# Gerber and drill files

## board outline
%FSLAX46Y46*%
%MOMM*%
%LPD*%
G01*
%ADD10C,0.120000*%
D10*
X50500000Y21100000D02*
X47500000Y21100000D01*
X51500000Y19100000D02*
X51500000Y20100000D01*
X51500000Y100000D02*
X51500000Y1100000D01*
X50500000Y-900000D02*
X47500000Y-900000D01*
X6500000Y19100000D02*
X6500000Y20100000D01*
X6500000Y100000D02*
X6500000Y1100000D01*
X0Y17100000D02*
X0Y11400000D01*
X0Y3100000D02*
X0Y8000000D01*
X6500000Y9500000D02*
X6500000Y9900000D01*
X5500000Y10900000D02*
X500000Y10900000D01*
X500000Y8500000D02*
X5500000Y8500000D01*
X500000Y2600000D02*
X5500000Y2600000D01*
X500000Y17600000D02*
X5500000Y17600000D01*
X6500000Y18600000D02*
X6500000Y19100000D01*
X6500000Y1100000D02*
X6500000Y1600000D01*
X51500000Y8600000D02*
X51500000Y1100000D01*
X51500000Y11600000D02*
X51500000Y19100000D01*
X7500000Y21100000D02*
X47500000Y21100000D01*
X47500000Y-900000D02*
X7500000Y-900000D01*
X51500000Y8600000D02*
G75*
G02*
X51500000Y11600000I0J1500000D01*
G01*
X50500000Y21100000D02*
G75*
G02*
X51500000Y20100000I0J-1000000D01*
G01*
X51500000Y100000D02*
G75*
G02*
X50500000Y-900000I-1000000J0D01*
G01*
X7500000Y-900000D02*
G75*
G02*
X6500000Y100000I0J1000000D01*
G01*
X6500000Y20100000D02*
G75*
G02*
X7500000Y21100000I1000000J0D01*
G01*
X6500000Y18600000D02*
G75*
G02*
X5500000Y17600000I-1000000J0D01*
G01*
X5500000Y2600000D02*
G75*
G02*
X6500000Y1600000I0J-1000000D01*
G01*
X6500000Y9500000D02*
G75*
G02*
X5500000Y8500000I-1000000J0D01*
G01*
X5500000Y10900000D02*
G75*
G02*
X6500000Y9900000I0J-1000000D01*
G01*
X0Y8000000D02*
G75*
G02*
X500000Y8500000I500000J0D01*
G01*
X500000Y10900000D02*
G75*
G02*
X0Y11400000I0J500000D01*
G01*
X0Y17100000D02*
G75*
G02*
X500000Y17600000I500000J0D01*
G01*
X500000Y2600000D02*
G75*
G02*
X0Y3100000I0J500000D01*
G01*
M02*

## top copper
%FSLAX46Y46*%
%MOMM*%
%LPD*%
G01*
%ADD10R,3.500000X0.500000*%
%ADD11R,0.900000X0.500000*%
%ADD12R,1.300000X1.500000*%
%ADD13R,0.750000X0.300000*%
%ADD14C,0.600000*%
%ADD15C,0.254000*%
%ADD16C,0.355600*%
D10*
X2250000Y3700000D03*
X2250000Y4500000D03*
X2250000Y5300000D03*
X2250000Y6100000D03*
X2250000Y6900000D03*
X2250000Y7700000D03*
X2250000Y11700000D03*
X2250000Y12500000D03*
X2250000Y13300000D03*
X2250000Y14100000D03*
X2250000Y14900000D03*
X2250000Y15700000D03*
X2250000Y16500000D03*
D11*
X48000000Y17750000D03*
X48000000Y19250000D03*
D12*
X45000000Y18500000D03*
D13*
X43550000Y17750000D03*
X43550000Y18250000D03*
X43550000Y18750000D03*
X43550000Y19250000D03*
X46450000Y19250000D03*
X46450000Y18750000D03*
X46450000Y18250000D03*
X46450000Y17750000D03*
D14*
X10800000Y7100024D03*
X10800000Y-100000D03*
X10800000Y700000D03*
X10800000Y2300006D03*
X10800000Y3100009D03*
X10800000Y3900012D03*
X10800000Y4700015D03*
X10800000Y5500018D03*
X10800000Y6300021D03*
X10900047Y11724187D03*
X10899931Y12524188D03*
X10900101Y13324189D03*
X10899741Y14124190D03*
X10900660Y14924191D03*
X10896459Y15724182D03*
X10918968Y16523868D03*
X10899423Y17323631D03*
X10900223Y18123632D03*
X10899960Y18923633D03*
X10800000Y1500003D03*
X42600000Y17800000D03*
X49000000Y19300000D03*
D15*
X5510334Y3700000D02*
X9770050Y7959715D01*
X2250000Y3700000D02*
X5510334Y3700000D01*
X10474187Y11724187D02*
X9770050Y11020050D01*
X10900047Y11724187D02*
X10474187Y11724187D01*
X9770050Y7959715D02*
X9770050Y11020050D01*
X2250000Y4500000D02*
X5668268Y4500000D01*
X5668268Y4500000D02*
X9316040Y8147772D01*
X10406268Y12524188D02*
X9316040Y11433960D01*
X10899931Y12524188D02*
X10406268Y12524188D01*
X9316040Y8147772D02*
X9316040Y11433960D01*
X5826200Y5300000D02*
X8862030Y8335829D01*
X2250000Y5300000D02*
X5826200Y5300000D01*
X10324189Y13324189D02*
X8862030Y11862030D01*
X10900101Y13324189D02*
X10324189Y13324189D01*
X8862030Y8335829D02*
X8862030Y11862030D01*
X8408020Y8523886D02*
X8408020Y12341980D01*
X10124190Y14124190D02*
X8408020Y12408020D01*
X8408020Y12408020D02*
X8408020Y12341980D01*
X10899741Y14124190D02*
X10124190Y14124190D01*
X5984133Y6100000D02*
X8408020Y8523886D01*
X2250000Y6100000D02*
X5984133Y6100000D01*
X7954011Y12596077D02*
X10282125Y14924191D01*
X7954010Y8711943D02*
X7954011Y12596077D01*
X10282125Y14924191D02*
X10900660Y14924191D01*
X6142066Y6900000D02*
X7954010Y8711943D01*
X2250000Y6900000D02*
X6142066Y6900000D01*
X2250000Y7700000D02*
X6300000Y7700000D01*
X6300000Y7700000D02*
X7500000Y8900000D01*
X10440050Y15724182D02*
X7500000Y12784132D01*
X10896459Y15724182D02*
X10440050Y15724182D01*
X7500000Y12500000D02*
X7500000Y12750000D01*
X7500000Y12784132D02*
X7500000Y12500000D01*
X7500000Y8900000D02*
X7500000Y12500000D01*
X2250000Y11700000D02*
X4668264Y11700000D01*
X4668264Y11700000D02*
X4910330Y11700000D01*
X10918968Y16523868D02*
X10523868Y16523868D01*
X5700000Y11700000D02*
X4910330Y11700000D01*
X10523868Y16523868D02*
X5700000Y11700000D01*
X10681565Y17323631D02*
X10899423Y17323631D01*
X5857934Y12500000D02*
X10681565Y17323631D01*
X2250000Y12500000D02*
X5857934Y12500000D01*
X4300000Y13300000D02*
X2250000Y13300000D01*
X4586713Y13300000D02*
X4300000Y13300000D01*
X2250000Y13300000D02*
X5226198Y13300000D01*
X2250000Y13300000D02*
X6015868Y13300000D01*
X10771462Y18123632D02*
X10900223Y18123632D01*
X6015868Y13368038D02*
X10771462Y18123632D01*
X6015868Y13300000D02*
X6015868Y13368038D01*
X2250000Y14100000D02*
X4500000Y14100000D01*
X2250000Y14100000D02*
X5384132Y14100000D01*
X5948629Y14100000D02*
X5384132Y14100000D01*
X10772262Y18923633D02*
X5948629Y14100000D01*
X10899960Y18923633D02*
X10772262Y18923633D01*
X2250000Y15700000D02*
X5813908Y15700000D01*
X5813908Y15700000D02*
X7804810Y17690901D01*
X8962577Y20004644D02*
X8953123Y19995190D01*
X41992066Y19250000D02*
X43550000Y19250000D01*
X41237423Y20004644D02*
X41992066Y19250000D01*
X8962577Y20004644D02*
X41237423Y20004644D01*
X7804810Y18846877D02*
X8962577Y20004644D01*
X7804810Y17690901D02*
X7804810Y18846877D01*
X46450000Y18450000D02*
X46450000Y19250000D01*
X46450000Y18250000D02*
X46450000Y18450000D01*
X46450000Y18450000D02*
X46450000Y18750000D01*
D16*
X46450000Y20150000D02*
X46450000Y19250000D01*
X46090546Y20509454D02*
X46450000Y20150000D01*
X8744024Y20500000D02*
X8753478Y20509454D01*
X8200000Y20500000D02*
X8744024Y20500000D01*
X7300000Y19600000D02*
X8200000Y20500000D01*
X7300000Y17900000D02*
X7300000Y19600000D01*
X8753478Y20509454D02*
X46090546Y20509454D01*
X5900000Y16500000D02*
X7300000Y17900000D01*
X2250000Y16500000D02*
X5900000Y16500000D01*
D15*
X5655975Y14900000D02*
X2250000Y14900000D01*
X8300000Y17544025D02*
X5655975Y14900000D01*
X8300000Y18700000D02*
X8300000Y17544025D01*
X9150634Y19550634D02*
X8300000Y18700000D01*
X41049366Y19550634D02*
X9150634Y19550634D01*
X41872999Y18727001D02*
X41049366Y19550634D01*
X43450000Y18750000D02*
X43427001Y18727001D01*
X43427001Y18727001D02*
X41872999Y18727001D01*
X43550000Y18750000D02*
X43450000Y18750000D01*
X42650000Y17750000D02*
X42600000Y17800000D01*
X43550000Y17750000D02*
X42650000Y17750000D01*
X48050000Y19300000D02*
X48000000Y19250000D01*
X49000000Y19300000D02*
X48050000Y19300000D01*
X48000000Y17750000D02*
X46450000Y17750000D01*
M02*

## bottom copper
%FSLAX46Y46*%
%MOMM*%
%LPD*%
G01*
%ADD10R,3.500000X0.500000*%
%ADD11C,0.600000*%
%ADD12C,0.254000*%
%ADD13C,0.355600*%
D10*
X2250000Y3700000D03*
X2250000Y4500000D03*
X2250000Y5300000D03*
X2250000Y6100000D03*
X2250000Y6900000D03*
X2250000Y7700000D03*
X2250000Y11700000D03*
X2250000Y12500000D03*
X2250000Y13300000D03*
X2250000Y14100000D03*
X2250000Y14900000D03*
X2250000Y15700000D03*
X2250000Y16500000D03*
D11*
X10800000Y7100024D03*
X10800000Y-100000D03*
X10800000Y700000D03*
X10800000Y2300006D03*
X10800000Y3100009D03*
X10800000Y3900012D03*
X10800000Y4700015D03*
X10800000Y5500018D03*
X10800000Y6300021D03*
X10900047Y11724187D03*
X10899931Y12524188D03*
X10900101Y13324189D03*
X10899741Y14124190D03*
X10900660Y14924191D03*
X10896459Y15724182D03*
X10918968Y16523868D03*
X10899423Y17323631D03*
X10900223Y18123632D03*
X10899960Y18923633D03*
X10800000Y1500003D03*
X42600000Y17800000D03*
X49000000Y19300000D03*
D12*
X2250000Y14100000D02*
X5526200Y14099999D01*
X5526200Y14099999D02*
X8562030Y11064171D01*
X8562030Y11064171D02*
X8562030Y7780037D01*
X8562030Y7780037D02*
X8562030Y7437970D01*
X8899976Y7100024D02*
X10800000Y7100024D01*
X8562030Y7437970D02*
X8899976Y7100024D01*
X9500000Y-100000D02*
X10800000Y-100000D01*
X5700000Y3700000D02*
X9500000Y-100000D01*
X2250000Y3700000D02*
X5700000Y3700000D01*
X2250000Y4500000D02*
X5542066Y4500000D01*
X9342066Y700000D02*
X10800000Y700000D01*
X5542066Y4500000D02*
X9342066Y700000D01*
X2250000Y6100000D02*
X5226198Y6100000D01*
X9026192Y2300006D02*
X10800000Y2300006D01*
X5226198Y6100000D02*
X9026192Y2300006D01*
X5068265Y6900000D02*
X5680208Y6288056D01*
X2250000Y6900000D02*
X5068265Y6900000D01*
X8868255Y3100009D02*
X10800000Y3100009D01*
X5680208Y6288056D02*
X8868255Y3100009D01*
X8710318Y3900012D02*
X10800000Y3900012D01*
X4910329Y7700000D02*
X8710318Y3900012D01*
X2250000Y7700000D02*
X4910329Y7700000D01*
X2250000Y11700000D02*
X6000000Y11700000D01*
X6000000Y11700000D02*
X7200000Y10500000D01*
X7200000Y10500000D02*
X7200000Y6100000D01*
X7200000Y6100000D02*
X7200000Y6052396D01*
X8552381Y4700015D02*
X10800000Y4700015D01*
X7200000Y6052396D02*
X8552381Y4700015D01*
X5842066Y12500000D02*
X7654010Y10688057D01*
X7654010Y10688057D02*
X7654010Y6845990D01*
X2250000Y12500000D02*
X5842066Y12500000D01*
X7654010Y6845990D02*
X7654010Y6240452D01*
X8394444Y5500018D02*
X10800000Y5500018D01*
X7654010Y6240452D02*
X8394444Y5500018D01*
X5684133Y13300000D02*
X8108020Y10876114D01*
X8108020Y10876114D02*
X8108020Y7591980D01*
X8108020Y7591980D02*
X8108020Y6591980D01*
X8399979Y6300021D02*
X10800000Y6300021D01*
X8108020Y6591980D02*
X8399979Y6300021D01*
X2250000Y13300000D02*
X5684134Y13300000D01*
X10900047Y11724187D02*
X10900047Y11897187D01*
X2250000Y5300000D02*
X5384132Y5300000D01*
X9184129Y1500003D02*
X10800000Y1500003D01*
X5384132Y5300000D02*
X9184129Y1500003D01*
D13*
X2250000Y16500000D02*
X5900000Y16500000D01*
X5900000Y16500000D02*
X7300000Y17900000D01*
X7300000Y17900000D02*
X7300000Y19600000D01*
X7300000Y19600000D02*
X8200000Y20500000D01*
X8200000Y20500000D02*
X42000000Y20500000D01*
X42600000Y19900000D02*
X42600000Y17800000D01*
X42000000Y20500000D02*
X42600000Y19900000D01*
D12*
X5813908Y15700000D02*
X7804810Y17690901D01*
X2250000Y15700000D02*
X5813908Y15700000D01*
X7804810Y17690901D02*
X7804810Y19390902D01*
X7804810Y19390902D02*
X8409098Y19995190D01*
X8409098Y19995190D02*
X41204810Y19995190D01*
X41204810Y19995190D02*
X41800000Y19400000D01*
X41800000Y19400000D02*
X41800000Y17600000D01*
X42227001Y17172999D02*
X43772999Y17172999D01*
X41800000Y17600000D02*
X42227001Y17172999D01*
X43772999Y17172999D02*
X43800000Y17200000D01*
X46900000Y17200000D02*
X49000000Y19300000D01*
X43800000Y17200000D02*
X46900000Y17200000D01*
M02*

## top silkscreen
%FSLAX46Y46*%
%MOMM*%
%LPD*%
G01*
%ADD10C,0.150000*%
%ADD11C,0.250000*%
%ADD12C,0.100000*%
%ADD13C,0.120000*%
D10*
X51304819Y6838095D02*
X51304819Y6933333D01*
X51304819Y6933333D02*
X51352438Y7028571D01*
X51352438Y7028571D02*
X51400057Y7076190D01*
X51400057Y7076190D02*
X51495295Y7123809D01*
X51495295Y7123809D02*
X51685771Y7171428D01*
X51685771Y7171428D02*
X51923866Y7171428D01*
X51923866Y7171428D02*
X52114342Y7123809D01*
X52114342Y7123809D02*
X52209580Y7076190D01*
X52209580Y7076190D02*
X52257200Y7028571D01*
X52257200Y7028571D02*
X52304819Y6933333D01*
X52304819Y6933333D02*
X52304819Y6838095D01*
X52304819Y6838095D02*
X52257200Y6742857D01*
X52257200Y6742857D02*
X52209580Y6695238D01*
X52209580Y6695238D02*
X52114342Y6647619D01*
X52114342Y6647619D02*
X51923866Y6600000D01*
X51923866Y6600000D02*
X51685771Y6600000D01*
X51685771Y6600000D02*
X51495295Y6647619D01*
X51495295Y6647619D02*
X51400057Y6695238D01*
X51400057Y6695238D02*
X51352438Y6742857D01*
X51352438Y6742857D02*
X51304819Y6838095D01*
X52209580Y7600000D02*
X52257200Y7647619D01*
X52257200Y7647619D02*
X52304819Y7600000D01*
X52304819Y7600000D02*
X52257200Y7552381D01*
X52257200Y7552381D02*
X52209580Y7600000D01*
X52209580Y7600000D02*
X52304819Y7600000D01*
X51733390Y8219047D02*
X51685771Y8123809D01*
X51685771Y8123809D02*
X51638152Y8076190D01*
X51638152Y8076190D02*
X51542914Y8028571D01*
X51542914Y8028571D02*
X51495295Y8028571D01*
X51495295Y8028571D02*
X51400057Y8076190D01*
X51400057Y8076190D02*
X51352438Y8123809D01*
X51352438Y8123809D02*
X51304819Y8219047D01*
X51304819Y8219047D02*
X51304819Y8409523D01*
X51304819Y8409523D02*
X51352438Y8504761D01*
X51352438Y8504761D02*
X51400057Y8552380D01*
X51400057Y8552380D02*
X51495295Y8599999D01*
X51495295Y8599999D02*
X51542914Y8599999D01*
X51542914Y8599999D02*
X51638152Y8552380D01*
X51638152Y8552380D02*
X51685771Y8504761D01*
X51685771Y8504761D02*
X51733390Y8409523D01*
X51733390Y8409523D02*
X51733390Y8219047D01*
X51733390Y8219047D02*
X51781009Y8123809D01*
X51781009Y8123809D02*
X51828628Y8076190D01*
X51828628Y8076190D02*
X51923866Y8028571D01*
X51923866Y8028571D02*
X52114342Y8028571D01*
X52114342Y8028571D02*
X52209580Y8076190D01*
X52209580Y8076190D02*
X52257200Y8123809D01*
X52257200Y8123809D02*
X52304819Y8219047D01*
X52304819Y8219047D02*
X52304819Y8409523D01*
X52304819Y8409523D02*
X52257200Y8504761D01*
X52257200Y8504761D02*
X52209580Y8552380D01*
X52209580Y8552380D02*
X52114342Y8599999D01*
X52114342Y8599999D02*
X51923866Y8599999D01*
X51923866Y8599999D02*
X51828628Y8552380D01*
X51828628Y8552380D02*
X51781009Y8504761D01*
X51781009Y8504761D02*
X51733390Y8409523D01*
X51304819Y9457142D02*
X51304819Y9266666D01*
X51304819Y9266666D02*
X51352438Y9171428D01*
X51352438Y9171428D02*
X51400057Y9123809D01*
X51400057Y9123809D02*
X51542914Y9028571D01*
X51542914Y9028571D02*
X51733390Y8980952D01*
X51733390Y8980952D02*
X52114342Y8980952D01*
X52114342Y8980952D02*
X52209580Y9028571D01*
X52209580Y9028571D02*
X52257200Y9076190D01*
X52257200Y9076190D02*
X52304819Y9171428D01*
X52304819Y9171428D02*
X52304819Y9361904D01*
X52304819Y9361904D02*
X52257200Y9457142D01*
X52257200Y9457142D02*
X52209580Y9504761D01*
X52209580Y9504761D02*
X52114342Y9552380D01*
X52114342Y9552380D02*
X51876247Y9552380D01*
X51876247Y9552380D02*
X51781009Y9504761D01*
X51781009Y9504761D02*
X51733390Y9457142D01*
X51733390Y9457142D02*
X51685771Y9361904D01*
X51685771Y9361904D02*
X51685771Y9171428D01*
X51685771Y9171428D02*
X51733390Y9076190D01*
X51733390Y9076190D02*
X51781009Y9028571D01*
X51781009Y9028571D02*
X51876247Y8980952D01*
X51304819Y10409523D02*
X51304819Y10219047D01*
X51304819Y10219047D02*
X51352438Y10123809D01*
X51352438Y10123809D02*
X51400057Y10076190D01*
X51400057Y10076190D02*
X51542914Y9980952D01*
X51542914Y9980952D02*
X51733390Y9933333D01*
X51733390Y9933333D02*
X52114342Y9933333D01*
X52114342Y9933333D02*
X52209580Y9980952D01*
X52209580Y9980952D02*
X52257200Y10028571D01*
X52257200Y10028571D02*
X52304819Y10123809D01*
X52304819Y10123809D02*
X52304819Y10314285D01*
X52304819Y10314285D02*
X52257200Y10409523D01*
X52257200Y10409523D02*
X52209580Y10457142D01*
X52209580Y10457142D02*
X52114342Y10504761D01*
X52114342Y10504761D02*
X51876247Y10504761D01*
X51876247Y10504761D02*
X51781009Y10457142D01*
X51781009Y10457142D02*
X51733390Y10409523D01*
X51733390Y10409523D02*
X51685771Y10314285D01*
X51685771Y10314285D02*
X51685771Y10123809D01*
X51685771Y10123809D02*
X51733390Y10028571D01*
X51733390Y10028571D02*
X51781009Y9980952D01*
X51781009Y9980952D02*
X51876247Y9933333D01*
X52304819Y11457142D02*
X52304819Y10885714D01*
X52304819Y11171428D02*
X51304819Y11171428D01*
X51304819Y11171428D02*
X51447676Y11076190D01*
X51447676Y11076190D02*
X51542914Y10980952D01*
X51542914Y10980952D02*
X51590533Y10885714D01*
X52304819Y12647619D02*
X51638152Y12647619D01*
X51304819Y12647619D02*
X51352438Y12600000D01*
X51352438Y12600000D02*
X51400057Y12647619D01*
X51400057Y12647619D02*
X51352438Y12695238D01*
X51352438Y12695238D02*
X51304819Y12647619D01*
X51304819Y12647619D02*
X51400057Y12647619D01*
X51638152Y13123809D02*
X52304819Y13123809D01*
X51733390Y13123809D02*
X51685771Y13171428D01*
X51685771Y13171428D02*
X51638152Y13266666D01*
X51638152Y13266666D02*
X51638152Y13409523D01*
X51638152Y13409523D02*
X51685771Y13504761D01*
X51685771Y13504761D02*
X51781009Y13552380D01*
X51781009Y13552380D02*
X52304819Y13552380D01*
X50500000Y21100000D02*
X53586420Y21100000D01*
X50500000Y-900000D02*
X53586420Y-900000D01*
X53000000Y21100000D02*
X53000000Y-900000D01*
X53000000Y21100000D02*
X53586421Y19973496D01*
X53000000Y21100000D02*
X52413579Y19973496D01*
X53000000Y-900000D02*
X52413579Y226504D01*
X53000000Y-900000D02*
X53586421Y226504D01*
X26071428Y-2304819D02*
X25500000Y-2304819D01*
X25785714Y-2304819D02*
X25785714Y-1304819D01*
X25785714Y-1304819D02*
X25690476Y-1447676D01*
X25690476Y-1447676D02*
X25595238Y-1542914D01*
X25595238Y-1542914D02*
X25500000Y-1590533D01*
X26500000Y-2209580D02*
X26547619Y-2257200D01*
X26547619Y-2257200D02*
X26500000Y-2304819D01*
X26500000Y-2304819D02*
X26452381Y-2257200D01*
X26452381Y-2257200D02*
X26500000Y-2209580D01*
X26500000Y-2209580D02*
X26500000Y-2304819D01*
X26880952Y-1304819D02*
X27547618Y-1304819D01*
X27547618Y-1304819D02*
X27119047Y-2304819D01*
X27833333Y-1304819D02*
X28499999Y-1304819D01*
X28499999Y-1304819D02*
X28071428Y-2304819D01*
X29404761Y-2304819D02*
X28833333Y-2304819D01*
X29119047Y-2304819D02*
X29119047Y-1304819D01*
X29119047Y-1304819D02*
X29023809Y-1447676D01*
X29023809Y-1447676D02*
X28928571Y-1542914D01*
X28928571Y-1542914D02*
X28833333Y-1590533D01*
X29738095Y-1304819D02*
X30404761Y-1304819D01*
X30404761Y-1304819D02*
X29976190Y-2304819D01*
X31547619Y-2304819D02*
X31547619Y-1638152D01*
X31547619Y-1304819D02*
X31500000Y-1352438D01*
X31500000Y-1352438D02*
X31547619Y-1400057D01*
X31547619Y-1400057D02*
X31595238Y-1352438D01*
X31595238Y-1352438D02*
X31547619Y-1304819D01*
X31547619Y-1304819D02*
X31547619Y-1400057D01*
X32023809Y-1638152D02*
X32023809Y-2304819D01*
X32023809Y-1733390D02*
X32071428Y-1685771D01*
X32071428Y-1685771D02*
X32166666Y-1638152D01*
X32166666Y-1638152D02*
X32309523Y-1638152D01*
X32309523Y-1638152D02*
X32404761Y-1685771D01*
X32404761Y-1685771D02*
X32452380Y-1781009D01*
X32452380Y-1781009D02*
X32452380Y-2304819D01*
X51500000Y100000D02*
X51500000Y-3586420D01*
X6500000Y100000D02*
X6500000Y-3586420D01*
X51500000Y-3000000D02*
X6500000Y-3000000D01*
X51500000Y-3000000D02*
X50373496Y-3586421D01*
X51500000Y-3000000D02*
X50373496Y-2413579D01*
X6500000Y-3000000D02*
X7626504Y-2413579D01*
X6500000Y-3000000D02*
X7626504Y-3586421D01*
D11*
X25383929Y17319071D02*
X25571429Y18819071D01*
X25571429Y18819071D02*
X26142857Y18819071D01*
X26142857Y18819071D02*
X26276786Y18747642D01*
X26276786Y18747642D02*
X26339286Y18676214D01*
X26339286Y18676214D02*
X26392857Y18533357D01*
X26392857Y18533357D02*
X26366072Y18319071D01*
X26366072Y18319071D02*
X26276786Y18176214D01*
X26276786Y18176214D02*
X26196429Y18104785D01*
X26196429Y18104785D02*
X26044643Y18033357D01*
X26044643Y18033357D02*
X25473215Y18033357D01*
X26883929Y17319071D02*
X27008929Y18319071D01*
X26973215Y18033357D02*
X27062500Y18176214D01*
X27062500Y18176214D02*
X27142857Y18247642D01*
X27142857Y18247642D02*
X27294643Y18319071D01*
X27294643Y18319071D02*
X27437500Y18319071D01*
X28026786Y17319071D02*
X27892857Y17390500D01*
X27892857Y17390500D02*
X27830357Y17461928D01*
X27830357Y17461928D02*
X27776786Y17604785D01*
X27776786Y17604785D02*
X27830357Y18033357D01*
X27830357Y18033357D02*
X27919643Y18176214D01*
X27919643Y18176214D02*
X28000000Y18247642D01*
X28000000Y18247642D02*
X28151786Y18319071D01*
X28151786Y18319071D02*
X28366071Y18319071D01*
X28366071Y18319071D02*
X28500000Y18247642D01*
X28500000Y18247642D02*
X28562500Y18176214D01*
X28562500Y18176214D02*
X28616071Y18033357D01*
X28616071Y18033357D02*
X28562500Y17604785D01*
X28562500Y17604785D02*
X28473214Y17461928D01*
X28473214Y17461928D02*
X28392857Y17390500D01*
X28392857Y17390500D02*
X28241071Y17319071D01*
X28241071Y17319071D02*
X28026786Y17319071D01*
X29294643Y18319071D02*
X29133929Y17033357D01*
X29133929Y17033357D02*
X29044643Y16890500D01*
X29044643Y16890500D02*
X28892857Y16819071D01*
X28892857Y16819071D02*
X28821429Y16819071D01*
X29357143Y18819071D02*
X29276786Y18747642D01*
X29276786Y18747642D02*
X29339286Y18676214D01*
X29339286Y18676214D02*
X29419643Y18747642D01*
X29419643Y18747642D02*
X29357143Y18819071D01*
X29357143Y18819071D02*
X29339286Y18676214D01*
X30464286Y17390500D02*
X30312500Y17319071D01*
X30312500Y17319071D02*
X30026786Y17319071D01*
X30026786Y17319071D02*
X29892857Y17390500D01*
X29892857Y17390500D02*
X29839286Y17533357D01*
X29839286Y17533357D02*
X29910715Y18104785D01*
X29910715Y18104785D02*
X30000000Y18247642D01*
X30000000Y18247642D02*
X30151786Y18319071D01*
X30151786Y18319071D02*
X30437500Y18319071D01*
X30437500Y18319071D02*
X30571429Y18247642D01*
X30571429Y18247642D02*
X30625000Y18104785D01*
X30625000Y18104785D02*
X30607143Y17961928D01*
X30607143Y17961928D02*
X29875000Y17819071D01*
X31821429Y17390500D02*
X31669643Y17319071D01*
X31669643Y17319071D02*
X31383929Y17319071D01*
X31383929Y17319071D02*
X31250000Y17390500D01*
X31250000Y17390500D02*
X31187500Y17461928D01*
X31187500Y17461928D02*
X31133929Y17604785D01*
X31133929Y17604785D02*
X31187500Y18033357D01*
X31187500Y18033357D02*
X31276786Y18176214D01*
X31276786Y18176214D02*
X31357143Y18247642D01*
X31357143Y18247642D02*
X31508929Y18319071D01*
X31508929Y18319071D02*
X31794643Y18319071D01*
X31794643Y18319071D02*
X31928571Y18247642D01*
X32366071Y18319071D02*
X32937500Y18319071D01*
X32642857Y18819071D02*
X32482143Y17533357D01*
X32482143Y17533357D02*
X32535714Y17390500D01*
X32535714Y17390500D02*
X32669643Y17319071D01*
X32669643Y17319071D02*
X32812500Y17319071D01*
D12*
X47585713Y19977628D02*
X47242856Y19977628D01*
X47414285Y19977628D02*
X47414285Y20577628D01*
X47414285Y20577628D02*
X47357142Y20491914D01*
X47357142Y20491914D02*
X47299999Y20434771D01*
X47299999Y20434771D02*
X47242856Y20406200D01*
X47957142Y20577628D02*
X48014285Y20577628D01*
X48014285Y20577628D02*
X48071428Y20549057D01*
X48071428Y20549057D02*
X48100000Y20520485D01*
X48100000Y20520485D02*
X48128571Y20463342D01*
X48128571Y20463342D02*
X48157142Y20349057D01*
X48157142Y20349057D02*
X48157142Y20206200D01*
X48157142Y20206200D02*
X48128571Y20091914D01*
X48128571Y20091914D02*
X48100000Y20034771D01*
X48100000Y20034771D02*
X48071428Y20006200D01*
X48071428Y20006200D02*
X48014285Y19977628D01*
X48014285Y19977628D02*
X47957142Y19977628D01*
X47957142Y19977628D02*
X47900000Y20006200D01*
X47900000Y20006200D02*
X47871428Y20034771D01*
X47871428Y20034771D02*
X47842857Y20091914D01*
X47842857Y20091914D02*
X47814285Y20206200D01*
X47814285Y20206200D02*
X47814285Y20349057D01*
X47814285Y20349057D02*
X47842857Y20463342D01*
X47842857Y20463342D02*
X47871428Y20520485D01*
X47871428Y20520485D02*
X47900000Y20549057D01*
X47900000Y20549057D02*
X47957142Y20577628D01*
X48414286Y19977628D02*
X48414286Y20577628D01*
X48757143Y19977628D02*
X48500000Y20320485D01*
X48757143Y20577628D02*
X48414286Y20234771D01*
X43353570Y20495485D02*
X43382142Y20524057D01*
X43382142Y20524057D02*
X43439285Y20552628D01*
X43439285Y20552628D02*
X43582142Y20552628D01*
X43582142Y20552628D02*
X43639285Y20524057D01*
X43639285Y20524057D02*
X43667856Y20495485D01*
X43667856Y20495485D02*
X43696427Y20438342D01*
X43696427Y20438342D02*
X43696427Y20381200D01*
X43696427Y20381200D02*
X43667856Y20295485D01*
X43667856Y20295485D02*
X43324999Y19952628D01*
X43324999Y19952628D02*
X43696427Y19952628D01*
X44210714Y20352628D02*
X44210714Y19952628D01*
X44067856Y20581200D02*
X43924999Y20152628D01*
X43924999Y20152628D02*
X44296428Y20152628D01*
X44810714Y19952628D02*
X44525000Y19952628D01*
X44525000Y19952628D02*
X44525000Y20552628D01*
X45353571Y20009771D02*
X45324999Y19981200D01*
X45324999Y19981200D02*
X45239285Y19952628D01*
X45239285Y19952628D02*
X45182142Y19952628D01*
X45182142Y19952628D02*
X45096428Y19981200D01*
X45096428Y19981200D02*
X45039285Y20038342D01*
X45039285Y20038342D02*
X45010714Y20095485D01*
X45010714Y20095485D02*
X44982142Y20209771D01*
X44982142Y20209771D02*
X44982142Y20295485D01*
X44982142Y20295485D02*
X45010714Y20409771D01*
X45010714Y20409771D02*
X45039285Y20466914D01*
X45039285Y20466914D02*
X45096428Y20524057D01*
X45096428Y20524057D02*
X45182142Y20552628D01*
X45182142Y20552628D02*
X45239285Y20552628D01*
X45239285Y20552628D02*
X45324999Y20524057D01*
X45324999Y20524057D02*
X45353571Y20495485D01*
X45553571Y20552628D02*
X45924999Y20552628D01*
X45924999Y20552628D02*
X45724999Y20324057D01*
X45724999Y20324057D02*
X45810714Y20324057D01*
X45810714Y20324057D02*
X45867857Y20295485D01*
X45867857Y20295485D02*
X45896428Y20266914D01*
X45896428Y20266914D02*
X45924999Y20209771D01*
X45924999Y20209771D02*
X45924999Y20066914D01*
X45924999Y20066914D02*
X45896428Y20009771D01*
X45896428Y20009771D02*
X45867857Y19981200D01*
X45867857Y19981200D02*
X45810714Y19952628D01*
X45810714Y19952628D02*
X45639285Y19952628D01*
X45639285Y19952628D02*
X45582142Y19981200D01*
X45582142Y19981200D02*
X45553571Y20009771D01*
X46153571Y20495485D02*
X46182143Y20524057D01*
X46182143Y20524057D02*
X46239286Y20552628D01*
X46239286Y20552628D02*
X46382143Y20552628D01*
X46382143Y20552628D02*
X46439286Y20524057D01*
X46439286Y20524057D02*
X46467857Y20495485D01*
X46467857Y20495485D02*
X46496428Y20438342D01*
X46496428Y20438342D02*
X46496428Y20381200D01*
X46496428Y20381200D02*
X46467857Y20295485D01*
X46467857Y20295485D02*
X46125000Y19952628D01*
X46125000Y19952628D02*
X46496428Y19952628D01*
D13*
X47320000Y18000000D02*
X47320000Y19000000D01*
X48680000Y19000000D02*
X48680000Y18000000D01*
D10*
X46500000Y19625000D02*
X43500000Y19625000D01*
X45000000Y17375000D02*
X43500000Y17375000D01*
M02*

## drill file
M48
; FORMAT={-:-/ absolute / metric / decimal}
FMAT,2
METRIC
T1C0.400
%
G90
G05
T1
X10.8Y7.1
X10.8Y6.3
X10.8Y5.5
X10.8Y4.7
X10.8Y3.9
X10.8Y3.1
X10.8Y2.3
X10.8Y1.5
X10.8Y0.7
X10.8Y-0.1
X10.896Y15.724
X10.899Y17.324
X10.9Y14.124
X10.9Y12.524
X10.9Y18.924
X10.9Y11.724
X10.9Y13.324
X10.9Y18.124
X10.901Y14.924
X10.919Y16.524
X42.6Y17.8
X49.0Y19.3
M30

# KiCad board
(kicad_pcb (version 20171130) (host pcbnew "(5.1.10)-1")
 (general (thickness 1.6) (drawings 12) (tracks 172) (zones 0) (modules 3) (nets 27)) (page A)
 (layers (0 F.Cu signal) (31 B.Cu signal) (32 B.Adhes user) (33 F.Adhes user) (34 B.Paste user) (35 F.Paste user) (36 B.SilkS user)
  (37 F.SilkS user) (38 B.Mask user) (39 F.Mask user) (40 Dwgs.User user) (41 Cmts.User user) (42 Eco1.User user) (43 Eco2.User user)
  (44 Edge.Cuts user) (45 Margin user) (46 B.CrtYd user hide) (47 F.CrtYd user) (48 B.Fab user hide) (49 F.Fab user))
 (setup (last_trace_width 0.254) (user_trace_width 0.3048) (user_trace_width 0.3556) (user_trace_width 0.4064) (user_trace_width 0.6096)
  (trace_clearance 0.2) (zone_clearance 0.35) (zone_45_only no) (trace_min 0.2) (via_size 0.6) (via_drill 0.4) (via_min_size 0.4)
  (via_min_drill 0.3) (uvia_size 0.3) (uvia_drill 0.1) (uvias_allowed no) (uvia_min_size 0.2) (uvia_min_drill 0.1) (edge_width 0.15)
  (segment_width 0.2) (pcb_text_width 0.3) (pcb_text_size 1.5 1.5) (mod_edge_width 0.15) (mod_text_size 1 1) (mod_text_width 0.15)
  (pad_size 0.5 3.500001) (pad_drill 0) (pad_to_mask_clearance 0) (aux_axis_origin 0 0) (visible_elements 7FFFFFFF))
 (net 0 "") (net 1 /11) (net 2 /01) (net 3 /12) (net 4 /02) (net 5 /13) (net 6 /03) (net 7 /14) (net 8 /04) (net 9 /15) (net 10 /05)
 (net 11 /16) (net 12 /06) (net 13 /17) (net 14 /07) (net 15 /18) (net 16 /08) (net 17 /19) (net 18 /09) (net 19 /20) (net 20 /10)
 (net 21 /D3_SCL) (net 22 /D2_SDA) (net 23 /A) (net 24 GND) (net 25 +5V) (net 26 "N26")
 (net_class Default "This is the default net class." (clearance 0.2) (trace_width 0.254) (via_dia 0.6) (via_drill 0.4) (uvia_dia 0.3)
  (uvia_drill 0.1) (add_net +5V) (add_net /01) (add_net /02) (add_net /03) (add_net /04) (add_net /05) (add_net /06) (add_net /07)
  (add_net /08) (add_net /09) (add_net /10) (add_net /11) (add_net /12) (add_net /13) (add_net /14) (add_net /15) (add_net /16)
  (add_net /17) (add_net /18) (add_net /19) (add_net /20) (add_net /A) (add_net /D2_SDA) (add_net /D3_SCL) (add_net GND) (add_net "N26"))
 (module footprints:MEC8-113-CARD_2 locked (layer F.Cu) (at 0 -0.1 90)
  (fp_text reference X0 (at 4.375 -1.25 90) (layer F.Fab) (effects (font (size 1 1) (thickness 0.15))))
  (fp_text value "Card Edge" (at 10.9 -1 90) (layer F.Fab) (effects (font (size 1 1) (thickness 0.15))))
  (fp_line (start 21 50.5) (end 21 47.5) (layer Edge.Cuts) (width 0.12))
  (fp_line (start 19 51.5) (end 20 51.5) (layer Edge.Cuts) (width 0.12))
  (fp_line (start 0 51.5) (end 1 51.5) (layer Edge.Cuts) (width 0.12))
  (fp_line (start -1 50.5) (end -1 47.5) (layer Edge.Cuts) (width 0.12))
  (fp_line (start 19 6.5) (end 20 6.5) (layer Edge.Cuts) (width 0.12))
  (fp_line (start 0 6.5) (end 1 6.5) (layer Edge.Cuts) (width 0.12))
  (fp_line (start 17 0) (end 11.3 0) (layer Edge.Cuts) (width 0.12))
  (fp_line (start 3 0) (end 7.9 0) (layer Edge.Cuts) (width 0.12))
  (fp_line (start 9.4 6.5) (end 9.8 6.5) (layer Edge.Cuts) (width 0.12))
  (fp_line (start 10.8 5.5) (end 10.8 0.5) (layer Edge.Cuts) (width 0.12))
  (fp_line (start 8.4 0.5) (end 8.4 5.5) (layer Edge.Cuts) (width 0.12))
  (fp_line (start 2.5 0.5) (end 2.5 5.5) (layer Edge.Cuts) (width 0.12))
  (fp_line (start 17.5 0.5) (end 17.5 5.5) (layer Edge.Cuts) (width 0.12))
  (fp_line (start 18.5 6.5) (end 19 6.5) (layer Edge.Cuts) (width 0.12))
  (fp_line (start 1 6.5) (end 1.5 6.5) (layer Edge.Cuts) (width 0.12))
  (fp_line (start 8.5 51.5) (end 1 51.5) (layer Edge.Cuts) (width 0.12))
  (fp_line (start 11.5 51.5) (end 19 51.5) (layer Edge.Cuts) (width 0.12))
  (fp_line (start 21 7.5) (end 21 47.5) (layer Edge.Cuts) (width 0.12))
  (fp_line (start -1 47.5) (end -1 7.5) (layer Edge.Cuts) (width 0.12))
  (fp_arc (start 10 51.5) (end 11.5 51.5) (angle -180) (layer Edge.Cuts) (width 0.12))
  (fp_arc (start 20 50.5) (end 20 51.5) (angle -90) (layer Edge.Cuts) (width 0.12))
  (fp_arc (start 0 50.5) (end -1 50.5) (angle -90) (layer Edge.Cuts) (width 0.12))
  (fp_arc (start 0 7.5) (end 0 6.5) (angle -90) (layer Edge.Cuts) (width 0.12))
  (fp_arc (start 20 7.5) (end 21 7.5) (angle -90) (layer Edge.Cuts) (width 0.12))
  (fp_arc (start 18.5 5.5) (end 17.5 5.5) (angle -90) (layer Edge.Cuts) (width 0.12))
  (fp_arc (start 1.5 5.5) (end 1.5 6.5) (angle -90) (layer Edge.Cuts) (width 0.12))
  (fp_arc (start 9.4 5.5) (end 8.4 5.5) (angle -90) (layer Edge.Cuts) (width 0.12))
  (fp_arc (start 9.8 5.5) (end 9.8 6.5) (angle -90) (layer Edge.Cuts) (width 0.12))
  (fp_arc (start 7.9 0.5) (end 8.4 0.5) (angle -90) (layer Edge.Cuts) (width 0.12))
  (fp_arc (start 11.3 0.5) (end 11.3 0) (angle -90) (layer Edge.Cuts) (width 0.12))
  (fp_arc (start 17 0.5) (end 17.5 0.5) (angle -90) (layer Edge.Cuts) (width 0.12))
  (fp_arc (start 3 0.5) (end 3 0) (angle -90) (layer Edge.Cuts) (width 0.12))
  (pad 14 smd rect (at 3.6 2.25 90) (size 0.5 3.5) (layers F.Cu F.Paste F.Mask) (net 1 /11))
  (pad 1 smd rect (at 3.6 2.25 90) (size 0.5 3.5) (layers B.Cu B.Paste B.Mask) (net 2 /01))
  (pad 15 smd rect (at 4.4 2.25 90) (size 0.5 3.5) (layers F.Cu F.Paste F.Mask) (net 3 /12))
  (pad 2 smd rect (at 4.4 2.25 90) (size 0.5 3.5) (layers B.Cu B.Paste B.Mask) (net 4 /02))
  (pad 16 smd rect (at 5.2 2.25 90) (size 0.5 3.5) (layers F.Cu F.Paste F.Mask) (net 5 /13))
  (pad 3 smd rect (at 5.2 2.25 90) (size 0.5 3.5) (layers B.Cu B.Paste B.Mask) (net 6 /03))
  (pad 17 smd rect (at 6 2.25 90) (size 0.5 3.5) (layers F.Cu F.Paste F.Mask) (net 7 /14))
  (pad 4 smd rect (at 6 2.25 90) (size 0.5 3.5) (layers B.Cu B.Paste B.Mask) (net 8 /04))
  (pad 18 smd rect (at 6.8 2.25 90) (size 0.5 3.5) (layers F.Cu F.Paste F.Mask) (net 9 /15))
  (pad 5 smd rect (at 6.8 2.25 90) (size 0.5 3.5) (layers B.Cu B.Paste B.Mask) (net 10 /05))
  (pad 19 smd rect (at 7.6 2.25 90) (size 0.5 3.5) (layers F.Cu F.Paste F.Mask) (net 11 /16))
  (pad 6 smd rect (at 7.6 2.25 90) (size 0.5 3.5) (layers B.Cu B.Paste B.Mask) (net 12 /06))
  (pad 20 smd rect (at 11.6 2.25 90) (size 0.5 3.5) (layers F.Cu F.Paste F.Mask) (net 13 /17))
  (pad 7 smd rect (at 11.6 2.25 90) (size 0.5 3.5) (layers B.Cu B.Paste B.Mask) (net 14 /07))
  (pad 21 smd rect (at 12.4 2.25 90) (size 0.5 3.5) (layers F.Cu F.Paste F.Mask) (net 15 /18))
  (pad 8 smd rect (at 12.4 2.25 90) (size 0.5 3.5) (layers B.Cu B.Paste B.Mask) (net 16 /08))
  (pad 22 smd rect (at 13.2 2.25 90) (size 0.5 3.5) (layers F.Cu F.Paste F.Mask) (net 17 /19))
  (pad 9 smd rect (at 13.2 2.25 90) (size 0.5 3.5) (layers B.Cu B.Paste B.Mask) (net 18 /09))
  (pad 23 smd rect (at 14 2.25 90) (size 0.5 3.5) (layers F.Cu F.Paste F.Mask) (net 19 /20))
  (pad 10 smd rect (at 14 2.25 90) (size 0.5 3.5) (layers B.Cu B.Paste B.Mask) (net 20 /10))
  (pad 24 smd rect (at 14.8 2.25 90) (size 0.5 3.5) (layers F.Cu F.Paste F.Mask) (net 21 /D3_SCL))
  (pad 11 smd rect (at 14.8 2.25 90) (size 0.5 3.5) (layers B.Cu B.Paste B.Mask))
  (pad 25 smd rect (at 15.6 2.25 90) (size 0.5 3.5) (layers F.Cu F.Paste F.Mask) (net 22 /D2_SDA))
  (pad 12 smd rect (at 15.6 2.25 90) (size 0.5 3.5) (layers B.Cu B.Paste B.Mask) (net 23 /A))
  (pad 26 smd rect (at 16.4 2.25 90) (size 0.5 3.5) (layers F.Cu F.Paste F.Mask) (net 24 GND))
  (pad 13 smd rect (at 16.4 2.25 90) (size 0.5 3.5) (layers B.Cu B.Paste B.Mask) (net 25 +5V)))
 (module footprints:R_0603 (layer F.Cu) (at 48 -18.5 90)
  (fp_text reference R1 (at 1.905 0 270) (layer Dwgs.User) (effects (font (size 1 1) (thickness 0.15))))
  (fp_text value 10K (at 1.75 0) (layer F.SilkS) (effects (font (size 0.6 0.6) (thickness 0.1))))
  (fp_line (start -0.5 -0.68) (end 0.5 -0.68) (layer F.SilkS) (width 0.12))
  (fp_line (start 0.5 0.68) (end -0.5 0.68) (layer F.SilkS) (width 0.12))
  (pad 1 smd rect (at -0.75 0 90) (size 0.5 0.9) (layers F.Cu F.Paste F.Mask) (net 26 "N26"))
  (pad 2 smd rect (at 0.75 0 90) (size 0.5 0.9) (layers F.Cu F.Paste F.Mask) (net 23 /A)))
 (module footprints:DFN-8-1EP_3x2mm (layer F.Cu) (at 45 -18.5 180)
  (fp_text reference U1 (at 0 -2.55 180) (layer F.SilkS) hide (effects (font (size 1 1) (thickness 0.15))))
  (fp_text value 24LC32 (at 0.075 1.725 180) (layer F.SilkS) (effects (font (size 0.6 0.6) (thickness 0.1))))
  (fp_line (start -1.5 1.125) (end 1.5 1.125) (layer F.SilkS) (width 0.15))
  (fp_line (start 0 -1.125) (end 1.5 -1.125) (layer F.SilkS) (width 0.15))
  (pad "" smd rect (at 0.325 0.375 180) (size 0.5 0.6) (layers F.Paste))
  (pad "" smd rect (at 0.325 -0.375 180) (size 0.5 0.6) (layers F.Paste))
  (pad "" smd rect (at -0.325 0.375 180) (size 0.5 0.6) (layers F.Paste))
  (pad "" smd rect (at -0.325 -0.375 180) (size 0.5 0.6) (layers F.Paste))
  (pad 9 smd rect (at 0 0 180) (size 1.3 1.5) (layers F.Cu F.Mask))
  (pad 8 smd rect (at 1.45 -0.75 180) (size 0.75 0.3) (layers F.Cu F.Paste F.Mask) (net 25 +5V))
  (pad 7 smd rect (at 1.45 -0.25 180) (size 0.75 0.3) (layers F.Cu F.Paste F.Mask))
  (pad 6 smd rect (at 1.45 0.25 180) (size 0.75 0.3) (layers F.Cu F.Paste F.Mask) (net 21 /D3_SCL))
  (pad 5 smd rect (at 1.45 0.75 180) (size 0.75 0.3) (layers F.Cu F.Paste F.Mask) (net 22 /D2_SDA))
  (pad 4 smd rect (at -1.45 0.75 180) (size 0.75 0.3) (layers F.Cu F.Paste F.Mask) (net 24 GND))
  (pad 3 smd rect (at -1.45 0.25 180) (size 0.75 0.3) (layers F.Cu F.Paste F.Mask) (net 24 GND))
  (pad 2 smd rect (at -1.45 -0.25 180) (size 0.75 0.3) (layers F.Cu F.Paste F.Mask) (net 24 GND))
  (pad 1 smd rect (at -1.45 -0.75 180) (size 0.75 0.3) (layers F.Cu F.Paste F.Mask) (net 26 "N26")))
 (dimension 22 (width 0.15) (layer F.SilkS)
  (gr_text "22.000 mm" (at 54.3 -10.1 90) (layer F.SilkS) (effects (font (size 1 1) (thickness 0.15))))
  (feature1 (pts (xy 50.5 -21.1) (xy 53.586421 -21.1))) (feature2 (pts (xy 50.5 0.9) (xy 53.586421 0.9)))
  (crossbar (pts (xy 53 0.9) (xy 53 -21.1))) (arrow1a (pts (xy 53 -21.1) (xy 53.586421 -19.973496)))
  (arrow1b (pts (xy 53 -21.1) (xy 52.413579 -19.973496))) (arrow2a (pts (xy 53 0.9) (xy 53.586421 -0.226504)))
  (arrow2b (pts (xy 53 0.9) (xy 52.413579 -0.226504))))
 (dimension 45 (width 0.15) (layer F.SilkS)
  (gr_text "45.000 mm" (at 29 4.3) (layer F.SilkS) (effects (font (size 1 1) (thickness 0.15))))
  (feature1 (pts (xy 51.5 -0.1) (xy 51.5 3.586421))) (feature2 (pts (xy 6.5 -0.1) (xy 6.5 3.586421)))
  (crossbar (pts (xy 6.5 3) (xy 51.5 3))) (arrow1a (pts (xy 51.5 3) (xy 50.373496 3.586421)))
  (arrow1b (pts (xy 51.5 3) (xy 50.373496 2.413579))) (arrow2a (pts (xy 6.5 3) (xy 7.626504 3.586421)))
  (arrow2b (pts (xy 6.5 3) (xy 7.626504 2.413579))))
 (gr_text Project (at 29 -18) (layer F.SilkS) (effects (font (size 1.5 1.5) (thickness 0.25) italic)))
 (segment (start 2.25 -14.1) (end 5.5262 -14.099999) (width 0.254) (layer B.Cu) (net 20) (status 10))
 (segment (start 5.5262 -14.099999) (end 8.56203 -11.064171) (width 0.254) (layer B.Cu) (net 20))
 (segment (start 8.56203 -11.064171) (end 8.56203 -7.780037) (width 0.254) (layer B.Cu) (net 20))
 (segment (start 8.56203 -7.780037) (end 8.56203 -7.43797) (width 0.254) (layer B.Cu) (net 20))
 (via (at 10.8 -7.100024) (size 0.6) (drill 0.4) (layers F.Cu B.Cu) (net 20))
 (segment (start 8.899976 -7.100024) (end 10.8 -7.100024) (width 0.254) (layer B.Cu) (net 20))
 (segment (start 8.56203 -7.43797) (end 8.899976 -7.100024) (width 0.254) (layer B.Cu) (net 20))
 (via (at 10.8 0.1) (size 0.6) (drill 0.4) (layers F.Cu B.Cu) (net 2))
 (segment (start 9.5 0.1) (end 10.8 0.1) (width 0.254) (layer B.Cu) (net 2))
 (segment (start 5.7 -3.7) (end 9.5 0.1) (width 0.254) (layer B.Cu) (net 2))
 (segment (start 2.25 -3.7) (end 5.7 -3.7) (width 0.254) (layer B.Cu) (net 2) (status 10))
 (segment (start 2.25 -4.5) (end 5.542066 -4.5) (width 0.254) (layer B.Cu) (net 4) (status 10))
 (via (at 10.8 -0.7) (size 0.6) (drill 0.4) (layers F.Cu B.Cu) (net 4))
 (segment (start 9.342066 -0.7) (end 10.8 -0.7) (width 0.254) (layer B.Cu) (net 4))
 (segment (start 5.542066 -4.5) (end 9.342066 -0.7) (width 0.254) (layer B.Cu) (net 4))
 (segment (start 2.25 -6.1) (end 5.226198 -6.1) (width 0.254) (layer B.Cu) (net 8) (status 10))
 (via (at 10.8 -2.300006) (size 0.6) (drill 0.4) (layers F.Cu B.Cu) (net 8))
 (segment (start 9.026192 -2.300006) (end 10.8 -2.300006) (width 0.254) (layer B.Cu) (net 8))
 (segment (start 5.226198 -6.1) (end 9.026192 -2.300006) (width 0.254) (layer B.Cu) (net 8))
 (segment (start 5.068265 -6.9) (end 5.680208 -6.288056) (width 0.254) (layer B.Cu) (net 10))
 (segment (start 2.25 -6.9) (end 5.068265 -6.9) (width 0.254) (layer B.Cu) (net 10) (status 10))
 (via (at 10.8 -3.100009) (size 0.6) (drill 0.4) (layers F.Cu B.Cu) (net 10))
 (segment (start 8.868255 -3.100009) (end 10.8 -3.100009) (width 0.254) (layer B.Cu) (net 10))
 (segment (start 5.680208 -6.288056) (end 8.868255 -3.100009) (width 0.254) (layer B.Cu) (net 10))
 (via (at 10.8 -3.900012) (size 0.6) (drill 0.4) (layers F.Cu B.Cu) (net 12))
 (segment (start 8.710318 -3.900012) (end 10.8 -3.900012) (width 0.254) (layer B.Cu) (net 12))
 (segment (start 4.910329 -7.7) (end 8.710318 -3.900012) (width 0.254) (layer B.Cu) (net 12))
 (segment (start 2.25 -7.7) (end 4.910329 -7.7) (width 0.254) (layer B.Cu) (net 12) (status 10))
 (segment (start 2.25 -11.7) (end 6 -11.7) (width 0.254) (layer B.Cu) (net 14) (status 10))
 (segment (start 6 -11.7) (end 7.2 -10.5) (width 0.254) (layer B.Cu) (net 14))
 (segment (start 7.2 -10.5) (end 7.2 -6.1) (width 0.254) (layer B.Cu) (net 14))
 (segment (start 7.2 -6.1) (end 7.2 -6.052396) (width 0.254) (layer B.Cu) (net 14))
 (via (at 10.8 -4.700015) (size 0.6) (drill 0.4) (layers F.Cu B.Cu) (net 14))
 (segment (start 8.552381 -4.700015) (end 10.8 -4.700015) (width 0.254) (layer B.Cu) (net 14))
 (segment (start 7.2 -6.052396) (end 8.552381 -4.700015) (width 0.254) (layer B.Cu) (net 14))
 (segment (start 5.842066 -12.5) (end 7.65401 -10.688057) (width 0.254) (layer B.Cu) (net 16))
 (segment (start 7.65401 -10.688057) (end 7.65401 -6.84599) (width 0.254) (layer B.Cu) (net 16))
 (segment (start 2.25 -12.5) (end 5.842066 -12.5) (width 0.254) (layer B.Cu) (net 16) (status 10))
 (segment (start 7.65401 -6.84599) (end 7.65401 -6.240452) (width 0.254) (layer B.Cu) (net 16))
 (segment (start 8.394444 -5.500018) (end 10.8 -5.500018) (width 0.254) (layer B.Cu) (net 16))
 (via (at 10.8 -5.500018) (size 0.6) (drill 0.4) (layers F.Cu B.Cu) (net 16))
 (segment (start 7.65401 -6.240452) (end 8.394444 -5.500018) (width 0.254) (layer B.Cu) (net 16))
 (segment (start 5.684133 -13.3) (end 8.10802 -10.876114) (width 0.254) (layer B.Cu) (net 18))
 (segment (start 8.10802 -10.876114) (end 8.10802 -7.59198) (width 0.254) (layer B.Cu) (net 18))
 (segment (start 8.10802 -7.59198) (end 8.10802 -6.59198) (width 0.254) (layer B.Cu) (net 18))
 (via (at 10.8 -6.300021) (size 0.6) (drill 0.4) (layers F.Cu B.Cu) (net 18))
 (segment (start 8.399979 -6.300021) (end 10.8 -6.300021) (width 0.254) (layer B.Cu) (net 18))
 (segment (start 8.10802 -6.59198) (end 8.399979 -6.300021) (width 0.254) (layer B.Cu) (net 18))
 (segment (start 2.25 -13.3) (end 5.684134 -13.3) (width 0.254) (layer B.Cu) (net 18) (status 10))
 (segment (start 5.510334 -3.7) (end 9.77005 -7.959715) (width 0.254) (layer F.Cu) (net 1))
 (segment (start 2.25 -3.7) (end 5.510334 -3.7) (width 0.254) (layer F.Cu) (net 1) (status 10))
 (via (at 10.900047 -11.724187) (size 0.6) (drill 0.4) (layers F.Cu B.Cu) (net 1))
 (segment (start 10.900047 -11.724187) (end 10.900047 -11.897187) (width 0.254) (layer B.Cu) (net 1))
 (segment (start 10.474187 -11.724187) (end 9.77005 -11.02005) (width 0.254) (layer F.Cu) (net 1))
 (segment (start 10.900047 -11.724187) (end 10.474187 -11.724187) (width 0.254) (layer F.Cu) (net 1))
 (segment (start 9.77005 -7.959715) (end 9.77005 -11.02005) (width 0.254) (layer F.Cu) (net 1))
 (segment (start 2.25 -4.5) (end 5.668268 -4.5) (width 0.254) (layer F.Cu) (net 3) (status 10))
 (segment (start 5.668268 -4.5) (end 9.31604 -8.147772) (width 0.254) (layer F.Cu) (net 3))
 (via (at 10.899931 -12.524188) (size 0.6) (drill 0.4) (layers F.Cu B.Cu) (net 3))
 (segment (start 10.406268 -12.524188) (end 9.31604 -11.43396) (width 0.254) (layer F.Cu) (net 3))
 (segment (start 10.899931 -12.524188) (end 10.406268 -12.524188) (width 0.254) (layer F.Cu) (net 3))
 (segment (start 9.31604 -8.147772) (end 9.31604 -11.43396) (width 0.254) (layer F.Cu) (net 3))
 (segment (start 5.8262 -5.3) (end 8.86203 -8.335829) (width 0.254) (layer F.Cu) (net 5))
 (segment (start 2.25 -5.3) (end 5.8262 -5.3) (width 0.254) (layer F.Cu) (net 5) (status 10))
 (via (at 10.900101 -13.324189) (size 0.6) (drill 0.4) (layers F.Cu B.Cu) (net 5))
 (segment (start 10.324189 -13.324189) (end 8.86203 -11.86203) (width 0.254) (layer F.Cu) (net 5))
 (segment (start 10.900101 -13.324189) (end 10.324189 -13.324189) (width 0.254) (layer F.Cu) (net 5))
 (segment (start 8.86203 -8.335829) (end 8.86203 -11.86203) (width 0.254) (layer F.Cu) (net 5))
 (segment (start 8.40802 -8.523886) (end 8.40802 -12.34198) (width 0.254) (layer F.Cu) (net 7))
 (segment (start 10.12419 -14.12419) (end 8.40802 -12.40802) (width 0.254) (layer F.Cu) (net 7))
 (segment (start 8.40802 -12.40802) (end 8.40802 -12.34198) (width 0.254) (layer F.Cu) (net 7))
 (segment (start 10.899741 -14.12419) (end 10.12419 -14.12419) (width 0.254) (layer F.Cu) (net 7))
 (segment (start 5.984133 -6.1) (end 8.40802 -8.523886) (width 0.254) (layer F.Cu) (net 7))
 (segment (start 2.25 -6.1) (end 5.984133 -6.1) (width 0.254) (layer F.Cu) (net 7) (status 10))
 (via (at 10.899741 -14.12419) (size 0.6) (drill 0.4) (layers F.Cu B.Cu) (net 7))
 (via (at 10.90066 -14.924191) (size 0.6) (drill 0.4) (layers F.Cu B.Cu) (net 9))
 (segment (start 7.954011 -12.596077) (end 10.282125 -14.924191) (width 0.254) (layer F.Cu) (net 9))
 (segment (start 7.95401 -8.711943) (end 7.954011 -12.596077) (width 0.254) (layer F.Cu) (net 9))
 (segment (start 10.282125 -14.924191) (end 10.90066 -14.924191) (width 0.254) (layer F.Cu) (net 9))
 (segment (start 6.142066 -6.9) (end 7.95401 -8.711943) (width 0.254) (layer F.Cu) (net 9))
 (segment (start 2.25 -6.9) (end 6.142066 -6.9) (width 0.254) (layer F.Cu) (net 9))
 (segment (start 2.25 -7.7) (end 6.3 -7.7) (width 0.254) (layer F.Cu) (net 11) (status 10))
 (segment (start 6.3 -7.7) (end 7.5 -8.9) (width 0.254) (layer F.Cu) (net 11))
 (via (at 10.896459 -15.724182) (size 0.6) (drill 0.4) (layers F.Cu B.Cu) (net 11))
 (segment (start 10.44005 -15.724182) (end 7.5 -12.784132) (width 0.254) (layer F.Cu) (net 11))
 (segment (start 10.896459 -15.724182) (end 10.44005 -15.724182) (width 0.254) (layer F.Cu) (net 11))
 (segment (start 7.5 -12.5) (end 7.5 -12.75) (width 0.254) (layer F.Cu) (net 11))
 (segment (start 7.5 -12.784132) (end 7.5 -12.5) (width 0.254) (layer F.Cu) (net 11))
 (segment (start 7.5 -8.9) (end 7.5 -12.5) (width 0.254) (layer F.Cu) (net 11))
 (segment (start 2.25 -11.7) (end 4.668264 -11.7) (width 0.254) (layer F.Cu) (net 13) (status 10))
 (segment (start 4.668264 -11.7) (end 4.91033 -11.7) (width 0.254) (layer F.Cu) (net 13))
 (via (at 10.918968 -16.523868) (size 0.6) (drill 0.4) (layers F.Cu B.Cu) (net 13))
 (segment (start 10.918968 -16.523868) (end 10.523868 -16.523868) (width 0.254) (layer F.Cu) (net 13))
 (segment (start 5.7 -11.7) (end 4.91033 -11.7) (width 0.254) (layer F.Cu) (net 13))
 (segment (start 10.523868 -16.523868) (end 5.7 -11.7) (width 0.254) (layer F.Cu) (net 13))
 (via (at 10.899423 -17.323631) (size 0.6) (drill 0.4) (layers F.Cu B.Cu) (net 15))
 (segment (start 10.681565 -17.323631) (end 10.899423 -17.323631) (width 0.254) (layer F.Cu) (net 15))
 (segment (start 5.857934 -12.5) (end 10.681565 -17.323631) (width 0.254) (layer F.Cu) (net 15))
 (segment (start 2.25 -12.5) (end 5.857934 -12.5) (width 0.254) (layer F.Cu) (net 15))
 (segment (start 4.3 -13.3) (end 2.25 -13.3) (width 0.254) (layer F.Cu) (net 17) (status 20))
 (segment (start 4.586713 -13.3) (end 4.3 -13.3) (width 0.254) (layer F.Cu) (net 17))
 (segment (start 2.25 -13.3) (end 5.226198 -13.3) (width 0.254) (layer F.Cu) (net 17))
 (segment (start 2.25 -13.3) (end 6.015868 -13.3) (width 0.254) (layer F.Cu) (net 17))
 (segment (start 10.771462 -18.123632) (end 10.900223 -18.123632) (width 0.254) (layer F.Cu) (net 17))
 (via (at 10.900223 -18.123632) (size 0.6) (drill 0.4) (layers F.Cu B.Cu) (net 17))
 (segment (start 6.015868 -13.368038) (end 10.771462 -18.123632) (width 0.254) (layer F.Cu) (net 17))
 (segment (start 6.015868 -13.3) (end 6.015868 -13.368038) (width 0.254) (layer F.Cu) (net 17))
 (segment (start 2.25 -14.1) (end 4.5 -14.1) (width 0.254) (layer F.Cu) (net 19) (status 10))
 (segment (start 2.25 -14.1) (end 5.384132 -14.1) (width 0.254) (layer F.Cu) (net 19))
 (via (at 10.89996 -18.923633) (size 0.6) (drill 0.4) (layers F.Cu B.Cu) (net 19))
 (segment (start 5.948629 -14.1) (end 5.384132 -14.1) (width 0.254) (layer F.Cu) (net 19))
 (segment (start 10.772262 -18.923633) (end 5.948629 -14.1) (width 0.254) (layer F.Cu) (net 19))
 (segment (start 10.89996 -18.923633) (end 10.772262 -18.923633) (width 0.254) (layer F.Cu) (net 19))
 (segment (start 2.25 -5.3) (end 5.384132 -5.3) (width 0.254) (layer B.Cu) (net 6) (status 10))
 (via (at 10.8 -1.500003) (size 0.6) (drill 0.4) (layers F.Cu B.Cu) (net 6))
 (segment (start 9.184129 -1.500003) (end 10.8 -1.500003) (width 0.254) (layer B.Cu) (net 6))
 (segment (start 5.384132 -5.3) (end 9.184129 -1.500003) (width 0.254) (layer B.Cu) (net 6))
 (segment (start 2.25 -15.7) (end 5.813908 -15.7) (width 0.254) (layer F.Cu) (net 22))
 (segment (start 5.813908 -15.7) (end 7.80481 -17.690901) (width 0.254) (layer F.Cu) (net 22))
 (segment (start 8.962577 -20.004644) (end 8.953123 -19.99519) (width 0.254) (layer F.Cu) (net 22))
 (segment (start 41.992066 -19.25) (end 43.55 -19.25) (width 0.254) (layer F.Cu) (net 22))
 (segment (start 41.237423 -20.004644) (end 41.992066 -19.25) (width 0.254) (layer F.Cu) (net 22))
 (segment (start 8.962577 -20.004644) (end 41.237423 -20.004644) (width 0.254) (layer F.Cu) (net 22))
 (segment (start 7.80481 -18.846877) (end 8.962577 -20.004644) (width 0.254) (layer F.Cu) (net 22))
 (segment (start 7.80481 -17.690901) (end 7.80481 -18.846877) (width 0.254) (layer F.Cu) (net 22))
 (segment (start 46.45 -18.45) (end 46.45 -19.25) (width 0.254) (layer F.Cu) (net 24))
 (segment (start 46.45 -18.25) (end 46.45 -18.45) (width 0.254) (layer F.Cu) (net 24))
 (segment (start 46.45 -18.45) (end 46.45 -18.75) (width 0.254) (layer F.Cu) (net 24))
 (segment (start 46.45 -20.15) (end 46.45 -19.25) (width 0.3556) (layer F.Cu) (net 24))
 (segment (start 46.090546 -20.509454) (end 46.45 -20.15) (width 0.3556) (layer F.Cu) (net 24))
 (segment (start 8.744024 -20.5) (end 8.753478 -20.509454) (width 0.3556) (layer F.Cu) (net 24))
 (segment (start 8.2 -20.5) (end 8.744024 -20.5) (width 0.3556) (layer F.Cu) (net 24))
 (segment (start 7.3 -19.6) (end 8.2 -20.5) (width 0.3556) (layer F.Cu) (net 24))
 (segment (start 7.3 -17.9) (end 7.3 -19.6) (width 0.3556) (layer F.Cu) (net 24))
 (segment (start 8.753478 -20.509454) (end 46.090546 -20.509454) (width 0.3556) (layer F.Cu) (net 24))
 (segment (start 5.9 -16.5) (end 7.3 -17.9) (width 0.3556) (layer F.Cu) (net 24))
 (segment (start 2.25 -16.5) (end 5.9 -16.5) (width 0.3556) (layer F.Cu) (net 24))
 (segment (start 5.655975 -14.9) (end 2.25 -14.9) (width 0.254) (layer F.Cu) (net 21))
 (segment (start 8.3 -17.544025) (end 5.655975 -14.9) (width 0.254) (layer F.Cu) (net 21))
 (segment (start 8.3 -18.7) (end 8.3 -17.544025) (width 0.254) (layer F.Cu) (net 21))
 (segment (start 9.150634 -19.550634) (end 8.3 -18.7) (width 0.254) (layer F.Cu) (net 21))
 (segment (start 41.049366 -19.550634) (end 9.150634 -19.550634) (width 0.254) (layer F.Cu) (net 21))
 (segment (start 41.872999 -18.727001) (end 41.049366 -19.550634) (width 0.254) (layer F.Cu) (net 21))
 (segment (start 43.45 -18.75) (end 43.427001 -18.727001) (width 0.254) (layer F.Cu) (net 21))
 (segment (start 43.427001 -18.727001) (end 41.872999 -18.727001) (width 0.254) (layer F.Cu) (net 21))
 (segment (start 43.55 -18.75) (end 43.45 -18.75) (width 0.254) (layer F.Cu) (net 21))
 (segment (start 2.25 -16.5) (end 5.9 -16.5) (width 0.3556) (layer B.Cu) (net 25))
 (segment (start 5.9 -16.5) (end 7.3 -17.9) (width 0.3556) (layer B.Cu) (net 25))
 (segment (start 7.3 -17.9) (end 7.3 -19.6) (width 0.3556) (layer B.Cu) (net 25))
 (segment (start 7.3 -19.6) (end 8.2 -20.5) (width 0.3556) (layer B.Cu) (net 25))
 (segment (start 8.2 -20.5) (end 42 -20.5) (width 0.3556) (layer B.Cu) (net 25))
 (via (at 42.6 -17.8) (size 0.6) (drill 0.4) (layers F.Cu B.Cu) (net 25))
 (segment (start 42.6 -19.9) (end 42.6 -17.8) (width 0.3556) (layer B.Cu) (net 25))
 (segment (start 42 -20.5) (end 42.6 -19.9) (width 0.3556) (layer B.Cu) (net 25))
 (segment (start 42.65 -17.75) (end 42.6 -17.8) (width 0.254) (layer F.Cu) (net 25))
 (segment (start 43.55 -17.75) (end 42.65 -17.75) (width 0.254) (layer F.Cu) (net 25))
 (segment (start 5.813908 -15.7) (end 7.80481 -17.690901) (width 0.254) (layer B.Cu) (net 23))
 (segment (start 2.25 -15.7) (end 5.813908 -15.7) (width 0.254) (layer B.Cu) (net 23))
 (segment (start 7.80481 -17.690901) (end 7.80481 -19.390902) (width 0.254) (layer B.Cu) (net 23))
 (segment (start 7.80481 -19.390902) (end 8.409098 -19.99519) (width 0.254) (layer B.Cu) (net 23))
 (segment (start 8.409098 -19.99519) (end 41.20481 -19.99519) (width 0.254) (layer B.Cu) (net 23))
 (segment (start 41.20481 -19.99519) (end 41.8 -19.4) (width 0.254) (layer B.Cu) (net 23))
 (segment (start 41.8 -19.4) (end 41.8 -17.6) (width 0.254) (layer B.Cu) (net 23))
 (segment (start 42.227001 -17.172999) (end 43.772999 -17.172999) (width 0.254) (layer B.Cu) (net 23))
 (segment (start 41.8 -17.6) (end 42.227001 -17.172999) (width 0.254) (layer B.Cu) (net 23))
 (segment (start 43.772999 -17.172999) (end 43.8 -17.2) (width 0.254) (layer B.Cu) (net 23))
 (via (at 49 -19.3) (size 0.6) (drill 0.4) (layers F.Cu B.Cu) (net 23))
 (segment (start 46.9 -17.2) (end 49 -19.3) (width 0.254) (layer B.Cu) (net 23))
 (segment (start 43.8 -17.2) (end 46.9 -17.2) (width 0.254) (layer B.Cu) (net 23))
 (segment (start 48.05 -19.3) (end 48 -19.25) (width 0.254) (layer F.Cu) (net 23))
 (segment (start 49 -19.3) (end 48.05 -19.3) (width 0.254) (layer F.Cu) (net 23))
 (segment (start 48 -17.75) (end 46.45 -17.75) (width 0.254) (layer F.Cu) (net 26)))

